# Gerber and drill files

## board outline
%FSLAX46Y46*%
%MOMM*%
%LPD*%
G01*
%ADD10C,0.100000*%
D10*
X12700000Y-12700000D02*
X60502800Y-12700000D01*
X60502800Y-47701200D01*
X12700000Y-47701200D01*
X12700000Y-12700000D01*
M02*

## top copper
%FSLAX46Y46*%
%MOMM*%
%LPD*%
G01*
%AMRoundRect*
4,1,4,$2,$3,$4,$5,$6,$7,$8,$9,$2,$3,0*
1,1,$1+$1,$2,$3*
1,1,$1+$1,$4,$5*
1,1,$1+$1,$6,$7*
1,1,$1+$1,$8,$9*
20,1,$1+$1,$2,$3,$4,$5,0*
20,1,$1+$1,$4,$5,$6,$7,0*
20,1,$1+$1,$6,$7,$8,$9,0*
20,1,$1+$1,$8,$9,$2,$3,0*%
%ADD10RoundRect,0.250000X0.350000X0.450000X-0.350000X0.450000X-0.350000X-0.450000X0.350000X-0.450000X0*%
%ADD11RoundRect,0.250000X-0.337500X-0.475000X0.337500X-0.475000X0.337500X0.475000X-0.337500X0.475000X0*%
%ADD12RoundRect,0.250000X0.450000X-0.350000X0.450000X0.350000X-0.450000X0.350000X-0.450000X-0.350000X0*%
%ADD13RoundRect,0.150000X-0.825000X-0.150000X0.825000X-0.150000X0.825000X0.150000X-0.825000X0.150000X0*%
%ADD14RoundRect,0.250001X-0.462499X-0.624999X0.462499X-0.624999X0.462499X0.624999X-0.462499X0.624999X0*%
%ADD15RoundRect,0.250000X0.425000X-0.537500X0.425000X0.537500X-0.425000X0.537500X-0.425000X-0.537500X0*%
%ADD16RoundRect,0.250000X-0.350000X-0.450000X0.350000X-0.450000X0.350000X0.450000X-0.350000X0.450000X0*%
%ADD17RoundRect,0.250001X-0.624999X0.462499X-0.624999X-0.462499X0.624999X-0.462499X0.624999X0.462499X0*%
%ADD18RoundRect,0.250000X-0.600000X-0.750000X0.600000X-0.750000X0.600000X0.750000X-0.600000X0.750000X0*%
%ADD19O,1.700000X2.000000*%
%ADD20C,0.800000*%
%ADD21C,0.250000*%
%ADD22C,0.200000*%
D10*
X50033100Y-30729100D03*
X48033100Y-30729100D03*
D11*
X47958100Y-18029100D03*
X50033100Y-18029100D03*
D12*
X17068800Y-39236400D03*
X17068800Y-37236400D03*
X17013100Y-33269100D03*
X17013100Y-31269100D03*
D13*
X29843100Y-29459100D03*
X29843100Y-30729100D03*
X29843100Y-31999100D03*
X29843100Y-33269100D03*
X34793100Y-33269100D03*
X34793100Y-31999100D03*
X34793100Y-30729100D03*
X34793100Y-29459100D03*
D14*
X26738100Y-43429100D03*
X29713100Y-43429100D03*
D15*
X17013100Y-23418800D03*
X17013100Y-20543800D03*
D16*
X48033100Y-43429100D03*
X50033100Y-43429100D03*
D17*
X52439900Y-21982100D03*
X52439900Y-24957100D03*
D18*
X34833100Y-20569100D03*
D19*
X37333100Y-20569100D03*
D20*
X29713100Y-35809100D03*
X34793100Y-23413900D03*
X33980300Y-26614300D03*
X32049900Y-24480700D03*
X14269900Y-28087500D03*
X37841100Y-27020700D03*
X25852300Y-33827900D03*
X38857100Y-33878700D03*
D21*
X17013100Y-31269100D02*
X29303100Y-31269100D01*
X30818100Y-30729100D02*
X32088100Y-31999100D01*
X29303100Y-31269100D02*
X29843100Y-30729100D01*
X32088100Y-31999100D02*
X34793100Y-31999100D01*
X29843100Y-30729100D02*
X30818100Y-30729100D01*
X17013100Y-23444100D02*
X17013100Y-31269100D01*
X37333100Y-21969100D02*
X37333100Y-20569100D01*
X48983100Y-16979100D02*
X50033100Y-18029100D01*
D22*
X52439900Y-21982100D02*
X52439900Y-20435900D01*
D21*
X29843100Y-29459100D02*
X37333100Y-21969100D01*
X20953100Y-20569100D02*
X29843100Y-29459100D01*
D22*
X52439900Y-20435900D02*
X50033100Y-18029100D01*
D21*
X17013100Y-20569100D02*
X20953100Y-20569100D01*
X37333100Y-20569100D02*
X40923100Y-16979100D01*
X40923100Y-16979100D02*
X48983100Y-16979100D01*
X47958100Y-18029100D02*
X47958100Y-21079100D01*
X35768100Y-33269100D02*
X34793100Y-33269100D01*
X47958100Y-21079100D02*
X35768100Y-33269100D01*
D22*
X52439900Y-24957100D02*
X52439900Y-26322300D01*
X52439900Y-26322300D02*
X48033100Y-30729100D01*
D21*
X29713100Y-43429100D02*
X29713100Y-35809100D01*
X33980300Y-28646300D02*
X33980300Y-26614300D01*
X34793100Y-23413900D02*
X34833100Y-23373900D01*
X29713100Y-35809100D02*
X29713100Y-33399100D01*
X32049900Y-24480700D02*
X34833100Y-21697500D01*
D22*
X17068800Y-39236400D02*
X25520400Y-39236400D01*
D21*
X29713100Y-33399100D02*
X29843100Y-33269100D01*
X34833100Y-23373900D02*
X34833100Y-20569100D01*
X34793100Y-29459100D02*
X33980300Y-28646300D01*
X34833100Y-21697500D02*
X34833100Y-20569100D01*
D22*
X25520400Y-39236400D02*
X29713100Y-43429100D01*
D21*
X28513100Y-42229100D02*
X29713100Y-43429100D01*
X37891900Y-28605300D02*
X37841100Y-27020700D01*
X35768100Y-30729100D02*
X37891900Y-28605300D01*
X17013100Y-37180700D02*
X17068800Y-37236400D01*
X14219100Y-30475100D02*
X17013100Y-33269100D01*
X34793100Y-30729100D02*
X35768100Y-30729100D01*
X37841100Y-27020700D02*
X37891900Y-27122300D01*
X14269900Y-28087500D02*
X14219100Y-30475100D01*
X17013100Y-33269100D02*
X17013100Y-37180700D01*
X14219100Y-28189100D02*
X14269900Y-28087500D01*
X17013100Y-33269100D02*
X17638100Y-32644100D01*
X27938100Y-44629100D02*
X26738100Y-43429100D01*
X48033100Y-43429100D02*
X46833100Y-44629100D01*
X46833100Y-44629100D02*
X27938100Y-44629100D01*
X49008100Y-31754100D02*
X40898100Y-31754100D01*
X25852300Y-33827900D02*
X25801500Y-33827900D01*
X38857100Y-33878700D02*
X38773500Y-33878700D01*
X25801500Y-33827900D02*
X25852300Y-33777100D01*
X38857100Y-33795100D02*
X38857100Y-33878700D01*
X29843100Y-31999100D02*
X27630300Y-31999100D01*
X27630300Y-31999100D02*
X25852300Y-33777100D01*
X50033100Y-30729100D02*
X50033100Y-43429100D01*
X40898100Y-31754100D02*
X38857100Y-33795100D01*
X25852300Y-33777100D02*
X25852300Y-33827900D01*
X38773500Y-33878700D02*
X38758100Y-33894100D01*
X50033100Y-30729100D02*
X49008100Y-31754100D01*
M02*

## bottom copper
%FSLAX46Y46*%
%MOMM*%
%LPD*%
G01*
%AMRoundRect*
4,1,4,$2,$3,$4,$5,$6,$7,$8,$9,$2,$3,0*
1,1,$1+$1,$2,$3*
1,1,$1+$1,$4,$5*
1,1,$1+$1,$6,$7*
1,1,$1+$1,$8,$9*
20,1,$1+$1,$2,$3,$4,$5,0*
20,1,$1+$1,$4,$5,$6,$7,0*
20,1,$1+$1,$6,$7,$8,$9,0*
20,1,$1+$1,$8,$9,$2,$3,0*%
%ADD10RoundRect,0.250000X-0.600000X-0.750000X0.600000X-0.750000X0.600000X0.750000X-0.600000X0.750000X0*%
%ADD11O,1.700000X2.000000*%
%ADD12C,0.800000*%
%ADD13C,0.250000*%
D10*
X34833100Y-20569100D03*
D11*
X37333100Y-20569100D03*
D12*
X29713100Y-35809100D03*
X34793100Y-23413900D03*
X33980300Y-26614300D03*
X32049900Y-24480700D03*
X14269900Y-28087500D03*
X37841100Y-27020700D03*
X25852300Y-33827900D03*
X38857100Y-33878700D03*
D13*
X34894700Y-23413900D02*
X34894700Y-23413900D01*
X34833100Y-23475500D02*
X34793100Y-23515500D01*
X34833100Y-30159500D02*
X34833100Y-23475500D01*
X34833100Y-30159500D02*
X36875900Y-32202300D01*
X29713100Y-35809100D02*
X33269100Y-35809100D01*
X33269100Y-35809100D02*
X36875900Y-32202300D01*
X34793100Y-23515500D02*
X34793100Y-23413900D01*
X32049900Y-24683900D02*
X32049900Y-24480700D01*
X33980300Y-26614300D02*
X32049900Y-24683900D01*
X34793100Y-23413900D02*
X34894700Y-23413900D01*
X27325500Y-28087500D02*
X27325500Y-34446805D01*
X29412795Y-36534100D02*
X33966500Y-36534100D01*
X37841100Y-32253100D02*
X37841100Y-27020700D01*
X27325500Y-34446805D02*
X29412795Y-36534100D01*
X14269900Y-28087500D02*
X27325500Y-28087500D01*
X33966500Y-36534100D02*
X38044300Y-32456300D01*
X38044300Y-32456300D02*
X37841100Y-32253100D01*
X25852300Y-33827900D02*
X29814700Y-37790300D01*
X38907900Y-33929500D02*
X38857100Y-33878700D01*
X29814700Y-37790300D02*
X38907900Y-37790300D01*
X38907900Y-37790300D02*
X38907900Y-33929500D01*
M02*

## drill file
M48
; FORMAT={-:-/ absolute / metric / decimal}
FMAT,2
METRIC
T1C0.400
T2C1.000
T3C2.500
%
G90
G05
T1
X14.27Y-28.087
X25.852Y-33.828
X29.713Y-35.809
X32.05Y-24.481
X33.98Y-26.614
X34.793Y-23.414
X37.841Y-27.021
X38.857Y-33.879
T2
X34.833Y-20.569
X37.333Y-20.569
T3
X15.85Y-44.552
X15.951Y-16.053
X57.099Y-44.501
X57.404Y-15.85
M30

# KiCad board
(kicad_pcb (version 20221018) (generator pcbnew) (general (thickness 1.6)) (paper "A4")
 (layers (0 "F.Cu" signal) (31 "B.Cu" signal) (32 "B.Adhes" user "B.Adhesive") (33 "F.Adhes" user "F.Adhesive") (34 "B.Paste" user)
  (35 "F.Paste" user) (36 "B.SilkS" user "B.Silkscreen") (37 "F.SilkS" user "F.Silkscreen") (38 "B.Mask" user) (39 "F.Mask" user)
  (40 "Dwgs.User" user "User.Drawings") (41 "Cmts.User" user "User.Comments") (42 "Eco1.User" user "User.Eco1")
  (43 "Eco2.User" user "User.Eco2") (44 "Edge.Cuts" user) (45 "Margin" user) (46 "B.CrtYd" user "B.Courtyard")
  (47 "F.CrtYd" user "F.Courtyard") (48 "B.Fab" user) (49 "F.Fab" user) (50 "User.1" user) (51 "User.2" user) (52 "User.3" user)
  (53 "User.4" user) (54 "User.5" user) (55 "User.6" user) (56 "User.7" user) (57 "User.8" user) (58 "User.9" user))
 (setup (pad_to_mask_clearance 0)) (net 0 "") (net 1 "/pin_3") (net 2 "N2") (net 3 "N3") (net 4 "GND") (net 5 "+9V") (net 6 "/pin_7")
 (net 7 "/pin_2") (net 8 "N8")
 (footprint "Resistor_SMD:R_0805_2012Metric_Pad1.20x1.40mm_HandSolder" (layer "F.Cu") (at 49.0331 30.7291 180)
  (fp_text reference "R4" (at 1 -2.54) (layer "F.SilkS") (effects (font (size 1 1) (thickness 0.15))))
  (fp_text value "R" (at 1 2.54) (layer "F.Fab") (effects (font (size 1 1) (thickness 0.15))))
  (pad "1" smd roundrect (at -1 0 180) (size 1.2 1.4) (layers "F.Cu" "F.Paste" "F.Mask") (roundrect_rratio 0.208333) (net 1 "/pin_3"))
  (pad "2" smd roundrect (at 1 0 180) (size 1.2 1.4) (layers "F.Cu" "F.Paste" "F.Mask") (roundrect_rratio 0.208333) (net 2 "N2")))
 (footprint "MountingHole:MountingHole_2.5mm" (layer "F.Cu") (at 15.8496 44.5516)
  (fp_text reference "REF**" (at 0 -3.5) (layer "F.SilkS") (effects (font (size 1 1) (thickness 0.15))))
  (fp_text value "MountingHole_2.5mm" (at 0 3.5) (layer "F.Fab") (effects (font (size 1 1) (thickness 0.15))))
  (pad "" np_thru_hole circle (at 0 0) (size 2.5 2.5) (drill 2.5) (layers "*.Cu" "*.Mask")))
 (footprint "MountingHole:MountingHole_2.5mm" (layer "F.Cu") (at 57.0992 44.5008)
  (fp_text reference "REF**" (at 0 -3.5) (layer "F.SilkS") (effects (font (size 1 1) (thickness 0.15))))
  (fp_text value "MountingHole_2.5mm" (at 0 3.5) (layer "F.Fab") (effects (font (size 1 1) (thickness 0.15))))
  (pad "" np_thru_hole circle (at 0 0) (size 2.5 2.5) (drill 2.5) (layers "*.Cu" "*.Mask")))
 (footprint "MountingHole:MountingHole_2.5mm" (layer "F.Cu") (at 15.9512 16.0528)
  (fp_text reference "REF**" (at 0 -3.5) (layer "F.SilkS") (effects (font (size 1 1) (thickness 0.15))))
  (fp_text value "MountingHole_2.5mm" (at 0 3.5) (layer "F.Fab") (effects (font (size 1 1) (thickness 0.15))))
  (pad "" np_thru_hole circle (at 0 0) (size 2.5 2.5) (drill 2.5) (layers "*.Cu" "*.Mask")))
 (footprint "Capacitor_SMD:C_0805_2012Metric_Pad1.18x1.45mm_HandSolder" (layer "F.Cu") (at 48.9956 18.0291)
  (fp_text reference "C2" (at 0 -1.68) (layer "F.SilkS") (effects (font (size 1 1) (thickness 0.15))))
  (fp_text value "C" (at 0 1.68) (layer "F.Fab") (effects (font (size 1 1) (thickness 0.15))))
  (pad "1" smd roundrect (at -1.0375 0) (size 1.175 1.45) (layers "F.Cu" "F.Paste" "F.Mask") (roundrect_rratio 0.212766) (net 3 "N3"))
  (pad "2" smd roundrect (at 1.0375 0) (size 1.175 1.45) (layers "F.Cu" "F.Paste" "F.Mask") (roundrect_rratio 0.212766) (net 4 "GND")))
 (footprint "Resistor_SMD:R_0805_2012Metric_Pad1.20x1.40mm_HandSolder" (layer "F.Cu") (at 17.0688 38.2364 90)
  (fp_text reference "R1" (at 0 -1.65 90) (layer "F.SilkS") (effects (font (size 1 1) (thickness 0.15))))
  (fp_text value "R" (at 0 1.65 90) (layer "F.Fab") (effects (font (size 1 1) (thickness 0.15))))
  (pad "1" smd roundrect (at -1 0 90) (size 1.2 1.4) (layers "F.Cu" "F.Paste" "F.Mask") (roundrect_rratio 0.208333) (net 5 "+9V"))
  (pad "2" smd roundrect (at 1 0 90) (size 1.2 1.4) (layers "F.Cu" "F.Paste" "F.Mask") (roundrect_rratio 0.208333) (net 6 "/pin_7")))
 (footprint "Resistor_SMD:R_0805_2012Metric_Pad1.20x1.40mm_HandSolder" (layer "F.Cu") (at 17.0131 32.2691 90)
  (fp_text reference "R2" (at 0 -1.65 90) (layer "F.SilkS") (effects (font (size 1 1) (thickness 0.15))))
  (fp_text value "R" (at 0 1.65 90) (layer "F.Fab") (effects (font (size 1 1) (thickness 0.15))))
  (pad "1" smd roundrect (at -1 0 90) (size 1.2 1.4) (layers "F.Cu" "F.Paste" "F.Mask") (roundrect_rratio 0.208333) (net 6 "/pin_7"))
  (pad "2" smd roundrect (at 1 0 90) (size 1.2 1.4) (layers "F.Cu" "F.Paste" "F.Mask") (roundrect_rratio 0.208333) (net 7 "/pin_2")))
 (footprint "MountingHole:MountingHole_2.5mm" (layer "F.Cu") (at 57.404 15.8496)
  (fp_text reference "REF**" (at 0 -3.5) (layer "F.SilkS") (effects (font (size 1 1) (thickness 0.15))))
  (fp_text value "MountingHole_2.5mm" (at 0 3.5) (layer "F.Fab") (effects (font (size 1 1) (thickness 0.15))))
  (pad "" np_thru_hole circle (at 0 0) (size 2.5 2.5) (drill 2.5) (layers "*.Cu" "*.Mask")))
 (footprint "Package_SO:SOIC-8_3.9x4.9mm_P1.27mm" (layer "F.Cu") (at 32.3181 31.3641)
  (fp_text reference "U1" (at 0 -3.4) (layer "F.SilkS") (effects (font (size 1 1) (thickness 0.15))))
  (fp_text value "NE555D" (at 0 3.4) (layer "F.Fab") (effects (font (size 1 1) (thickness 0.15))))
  (pad "1" smd roundrect (at -2.475 -1.905) (size 1.95 0.6) (layers "F.Cu" "F.Paste" "F.Mask") (roundrect_rratio 0.25) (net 4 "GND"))
  (pad "2" smd roundrect (at -2.475 -0.635) (size 1.95 0.6) (layers "F.Cu" "F.Paste" "F.Mask") (roundrect_rratio 0.25) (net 7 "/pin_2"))
  (pad "3" smd roundrect (at -2.475 0.635) (size 1.95 0.6) (layers "F.Cu" "F.Paste" "F.Mask") (roundrect_rratio 0.25) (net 1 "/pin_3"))
  (pad "4" smd roundrect (at -2.475 1.905) (size 1.95 0.6) (layers "F.Cu" "F.Paste" "F.Mask") (roundrect_rratio 0.25) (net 5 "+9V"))
  (pad "5" smd roundrect (at 2.475 1.905) (size 1.95 0.6) (layers "F.Cu" "F.Paste" "F.Mask") (roundrect_rratio 0.25) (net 3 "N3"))
  (pad "6" smd roundrect (at 2.475 0.635) (size 1.95 0.6) (layers "F.Cu" "F.Paste" "F.Mask") (roundrect_rratio 0.25) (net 7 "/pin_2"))
  (pad "7" smd roundrect (at 2.475 -0.635) (size 1.95 0.6) (layers "F.Cu" "F.Paste" "F.Mask") (roundrect_rratio 0.25) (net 6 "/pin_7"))
  (pad "8" smd roundrect (at 2.475 -1.905) (size 1.95 0.6) (layers "F.Cu" "F.Paste" "F.Mask") (roundrect_rratio 0.25) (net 5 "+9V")))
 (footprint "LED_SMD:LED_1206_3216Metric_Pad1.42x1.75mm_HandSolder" (layer "F.Cu") (at 28.2256 43.4291)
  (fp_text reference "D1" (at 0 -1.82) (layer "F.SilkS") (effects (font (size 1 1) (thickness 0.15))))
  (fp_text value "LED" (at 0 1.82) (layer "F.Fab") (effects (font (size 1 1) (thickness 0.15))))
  (pad "1" smd roundrect (at -1.4875 0) (size 1.425 1.75) (layers "F.Cu" "F.Paste" "F.Mask") (roundrect_rratio 0.175439) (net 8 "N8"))
  (pad "2" smd roundrect (at 1.4875 0) (size 1.425 1.75) (layers "F.Cu" "F.Paste" "F.Mask") (roundrect_rratio 0.175439) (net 5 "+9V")))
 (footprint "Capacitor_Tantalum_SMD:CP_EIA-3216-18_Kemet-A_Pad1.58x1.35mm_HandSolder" (layer "F.Cu") (at 17.0131 21.9813 90)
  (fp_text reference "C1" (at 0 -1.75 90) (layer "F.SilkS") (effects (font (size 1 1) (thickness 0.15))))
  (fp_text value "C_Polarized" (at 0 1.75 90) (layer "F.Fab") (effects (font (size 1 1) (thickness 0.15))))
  (pad "1" smd roundrect (at -1.4375 0 90) (size 1.575 1.35) (layers "F.Cu" "F.Paste" "F.Mask") (roundrect_rratio 0.185185) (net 7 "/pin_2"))
  (pad "2" smd roundrect (at 1.4375 0 90) (size 1.575 1.35) (layers "F.Cu" "F.Paste" "F.Mask") (roundrect_rratio 0.185185) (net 4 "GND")))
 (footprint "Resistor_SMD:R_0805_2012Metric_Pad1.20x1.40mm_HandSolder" (layer "F.Cu") (at 49.0331 43.4291)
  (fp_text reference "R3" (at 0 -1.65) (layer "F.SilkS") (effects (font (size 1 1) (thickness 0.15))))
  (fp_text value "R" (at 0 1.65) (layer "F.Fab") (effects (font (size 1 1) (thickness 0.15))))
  (pad "1" smd roundrect (at -1 0) (size 1.2 1.4) (layers "F.Cu" "F.Paste" "F.Mask") (roundrect_rratio 0.208333) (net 8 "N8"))
  (pad "2" smd roundrect (at 1 0) (size 1.2 1.4) (layers "F.Cu" "F.Paste" "F.Mask") (roundrect_rratio 0.208333) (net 1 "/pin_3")))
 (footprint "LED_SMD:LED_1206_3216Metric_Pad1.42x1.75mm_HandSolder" (layer "F.Cu") (at 52.4399 23.4696 -90)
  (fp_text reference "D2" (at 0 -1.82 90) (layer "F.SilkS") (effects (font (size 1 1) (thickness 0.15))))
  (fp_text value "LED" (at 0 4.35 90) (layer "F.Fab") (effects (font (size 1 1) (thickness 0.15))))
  (pad "1" smd roundrect (at -1.4875 0 270) (size 1.425 1.75) (layers "F.Cu" "F.Paste" "F.Mask") (roundrect_rratio 0.175439) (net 4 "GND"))
  (pad "2" smd roundrect (at 1.4875 0 270) (size 1.425 1.75) (layers "F.Cu" "F.Paste" "F.Mask") (roundrect_rratio 0.175439) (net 2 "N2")))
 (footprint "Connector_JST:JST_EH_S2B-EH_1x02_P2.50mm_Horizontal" (layer "F.Cu") (at 34.8331 20.5691)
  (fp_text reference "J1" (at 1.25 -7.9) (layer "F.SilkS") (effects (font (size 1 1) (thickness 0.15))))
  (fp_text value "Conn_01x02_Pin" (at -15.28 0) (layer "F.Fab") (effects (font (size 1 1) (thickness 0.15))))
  (pad "1" thru_hole roundrect (at 0 0) (size 1.7 2) (drill 1) (layers "*.Cu" "*.Mask") (roundrect_rratio 0.147059) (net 5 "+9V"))
  (pad "2" thru_hole oval (at 2.5 0) (size 1.7 2) (drill 1) (layers "*.Cu" "*.Mask") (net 4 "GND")))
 (gr_rect (start 12.7 12.7) (end 60.5028 47.7012) (stroke (width 0.1) (type default)) (fill none) (layer "Edge.Cuts"))
 (segment (start 17.0131 31.2691) (end 29.3031 31.2691) (width 0.25) (layer "F.Cu") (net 7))
 (segment (start 30.8181 30.7291) (end 32.0881 31.9991) (width 0.25) (layer "F.Cu") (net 7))
 (segment (start 29.3031 31.2691) (end 29.8431 30.7291) (width 0.25) (layer "F.Cu") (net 7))
 (segment (start 32.0881 31.9991) (end 34.7931 31.9991) (width 0.25) (layer "F.Cu") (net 7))
 (segment (start 29.8431 30.7291) (end 30.8181 30.7291) (width 0.25) (layer "F.Cu") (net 7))
 (segment (start 17.0131 23.4441) (end 17.0131 31.2691) (width 0.25) (layer "F.Cu") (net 7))
 (segment (start 37.3331 21.9691) (end 37.3331 20.5691) (width 0.25) (layer "F.Cu") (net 4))
 (segment (start 48.9831 16.9791) (end 50.0331 18.0291) (width 0.25) (layer "F.Cu") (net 4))
 (segment (start 52.4399 21.9821) (end 52.4399 20.4359) (width 0.2) (layer "F.Cu") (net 4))
 (segment (start 29.8431 29.4591) (end 37.3331 21.9691) (width 0.25) (layer "F.Cu") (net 4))
 (segment (start 20.9531 20.5691) (end 29.8431 29.4591) (width 0.25) (layer "F.Cu") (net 4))
 (segment (start 52.4399 20.4359) (end 50.0331 18.0291) (width 0.2) (layer "F.Cu") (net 4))
 (segment (start 17.0131 20.5691) (end 20.9531 20.5691) (width 0.25) (layer "F.Cu") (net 4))
 (segment (start 37.3331 20.5691) (end 40.9231 16.9791) (width 0.25) (layer "F.Cu") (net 4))
 (segment (start 40.9231 16.9791) (end 48.9831 16.9791) (width 0.25) (layer "F.Cu") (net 4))
 (segment (start 47.9581 18.0291) (end 47.9581 21.0791) (width 0.25) (layer "F.Cu") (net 3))
 (segment (start 35.7681 33.2691) (end 34.7931 33.2691) (width 0.25) (layer "F.Cu") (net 3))
 (segment (start 47.9581 21.0791) (end 35.7681 33.2691) (width 0.25) (layer "F.Cu") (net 3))
 (segment (start 52.4399 24.9571) (end 52.4399 26.3223) (width 0.2) (layer "F.Cu") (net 2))
 (segment (start 52.4399 26.3223) (end 48.0331 30.7291) (width 0.2) (layer "F.Cu") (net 2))
 (segment (start 29.7131 43.4291) (end 29.7131 35.8091) (width 0.25) (layer "F.Cu") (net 5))
 (segment (start 33.9803 28.6463) (end 33.9803 26.6143) (width 0.25) (layer "F.Cu") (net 5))
 (segment (start 34.7931 23.4139) (end 34.8331 23.3739) (width 0.25) (layer "F.Cu") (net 5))
 (segment (start 29.7131 35.8091) (end 29.7131 33.3991) (width 0.25) (layer "F.Cu") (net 5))
 (segment (start 32.0499 24.4807) (end 34.8331 21.6975) (width 0.25) (layer "F.Cu") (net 5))
 (segment (start 17.0688 39.2364) (end 25.5204 39.2364) (width 0.2) (layer "F.Cu") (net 5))
 (segment (start 29.7131 33.3991) (end 29.8431 33.2691) (width 0.25) (layer "F.Cu") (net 5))
 (segment (start 34.8331 23.3739) (end 34.8331 20.5691) (width 0.25) (layer "F.Cu") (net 5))
 (segment (start 34.7931 29.4591) (end 33.9803 28.6463) (width 0.25) (layer "F.Cu") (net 5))
 (segment (start 34.8331 21.6975) (end 34.8331 20.5691) (width 0.25) (layer "F.Cu") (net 5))
 (segment (start 25.5204 39.2364) (end 29.7131 43.4291) (width 0.2) (layer "F.Cu") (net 5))
 (segment (start 28.5131 42.2291) (end 29.7131 43.4291) (width 0.25) (layer "F.Cu") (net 5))
 (via (at 29.7131 35.8091) (size 0.8) (drill 0.4) (layers "F.Cu" "B.Cu") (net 5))
 (via (at 34.7931 23.4139) (size 0.8) (drill 0.4) (layers "F.Cu" "B.Cu") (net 5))
 (via (at 33.9803 26.6143) (size 0.8) (drill 0.4) (layers "F.Cu" "B.Cu") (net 5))
 (via (at 32.0499 24.4807) (size 0.8) (drill 0.4) (layers "F.Cu" "B.Cu") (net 5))
 (segment (start 34.8947 23.4139) (end 34.8947 23.4139) (width 0.25) (layer "B.Cu") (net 5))
 (segment (start 34.8331 23.4755) (end 34.7931 23.5155) (width 0.25) (layer "B.Cu") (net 5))
 (segment (start 34.8331 30.1595) (end 34.8331 23.4755) (width 0.25) (layer "B.Cu") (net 5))
 (segment (start 34.8331 30.1595) (end 36.8759 32.2023) (width 0.25) (layer "B.Cu") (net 5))
 (segment (start 29.7131 35.8091) (end 33.2691 35.8091) (width 0.25) (layer "B.Cu") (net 5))
 (segment (start 33.2691 35.8091) (end 36.8759 32.2023) (width 0.25) (layer "B.Cu") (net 5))
 (segment (start 34.7931 23.5155) (end 34.7931 23.4139) (width 0.25) (layer "B.Cu") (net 5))
 (segment (start 32.0499 24.6839) (end 32.0499 24.4807) (width 0.25) (layer "B.Cu") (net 5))
 (segment (start 33.9803 26.6143) (end 32.0499 24.6839) (width 0.25) (layer "B.Cu") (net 5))
 (segment (start 34.7931 23.4139) (end 34.8947 23.4139) (width 0.25) (layer "B.Cu") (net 5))
 (segment (start 37.8919 28.6053) (end 37.8411 27.0207) (width 0.25) (layer "F.Cu") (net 6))
 (segment (start 35.7681 30.7291) (end 37.8919 28.6053) (width 0.25) (layer "F.Cu") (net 6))
 (segment (start 17.0131 37.1807) (end 17.0688 37.2364) (width 0.25) (layer "F.Cu") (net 6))
 (segment (start 14.2191 30.4751) (end 17.0131 33.2691) (width 0.25) (layer "F.Cu") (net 6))
 (segment (start 34.7931 30.7291) (end 35.7681 30.7291) (width 0.25) (layer "F.Cu") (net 6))
 (segment (start 37.8411 27.0207) (end 37.8919 27.1223) (width 0.25) (layer "F.Cu") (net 6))
 (segment (start 14.2699 28.0875) (end 14.2191 30.4751) (width 0.25) (layer "F.Cu") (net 6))
 (segment (start 17.0131 33.2691) (end 17.0131 37.1807) (width 0.25) (layer "F.Cu") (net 6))
 (segment (start 14.2191 28.1891) (end 14.2699 28.0875) (width 0.25) (layer "F.Cu") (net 6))
 (segment (start 17.0131 33.2691) (end 17.6381 32.6441) (width 0.25) (layer "F.Cu") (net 6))
 (via (at 14.2699 28.0875) (size 0.8) (drill 0.4) (layers "F.Cu" "B.Cu") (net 6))
 (via (at 37.8411 27.0207) (size 0.8) (drill 0.4) (layers "F.Cu" "B.Cu") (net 6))
 (segment (start 27.3255 28.0875) (end 27.3255 34.446805) (width 0.25) (layer "B.Cu") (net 6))
 (segment (start 29.412795 36.5341) (end 33.9665 36.5341) (width 0.25) (layer "B.Cu") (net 6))
 (segment (start 37.8411 32.2531) (end 37.8411 27.0207) (width 0.25) (layer "B.Cu") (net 6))
 (segment (start 27.3255 34.446805) (end 29.412795 36.5341) (width 0.25) (layer "B.Cu") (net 6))
 (segment (start 14.2699 28.0875) (end 27.3255 28.0875) (width 0.25) (layer "B.Cu") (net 6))
 (segment (start 33.9665 36.5341) (end 38.0443 32.4563) (width 0.25) (layer "B.Cu") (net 6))
 (segment (start 38.0443 32.4563) (end 37.8411 32.2531) (width 0.25) (layer "B.Cu") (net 6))
 (segment (start 27.9381 44.6291) (end 26.7381 43.4291) (width 0.25) (layer "F.Cu") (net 8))
 (segment (start 48.0331 43.4291) (end 46.8331 44.6291) (width 0.25) (layer "F.Cu") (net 8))
 (segment (start 46.8331 44.6291) (end 27.9381 44.6291) (width 0.25) (layer "F.Cu") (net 8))
 (segment (start 49.0081 31.7541) (end 40.8981 31.7541) (width 0.25) (layer "F.Cu") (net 1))
 (segment (start 25.8523 33.8279) (end 25.8015 33.8279) (width 0.25) (layer "F.Cu") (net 1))
 (segment (start 38.8571 33.8787) (end 38.7735 33.8787) (width 0.25) (layer "F.Cu") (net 1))
 (segment (start 25.8015 33.8279) (end 25.8523 33.7771) (width 0.25) (layer "F.Cu") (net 1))
 (segment (start 38.8571 33.7951) (end 38.8571 33.8787) (width 0.25) (layer "F.Cu") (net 1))
 (segment (start 29.8431 31.9991) (end 27.6303 31.9991) (width 0.25) (layer "F.Cu") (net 1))
 (segment (start 27.6303 31.9991) (end 25.8523 33.7771) (width 0.25) (layer "F.Cu") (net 1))
 (segment (start 50.0331 30.7291) (end 50.0331 43.4291) (width 0.25) (layer "F.Cu") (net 1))
 (segment (start 40.8981 31.7541) (end 38.8571 33.7951) (width 0.25) (layer "F.Cu") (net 1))
 (segment (start 25.8523 33.7771) (end 25.8523 33.8279) (width 0.25) (layer "F.Cu") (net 1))
 (segment (start 38.7735 33.8787) (end 38.7581 33.8941) (width 0.25) (layer "F.Cu") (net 1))
 (segment (start 50.0331 30.7291) (end 49.0081 31.7541) (width 0.25) (layer "F.Cu") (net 1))
 (via (at 25.8523 33.8279) (size 0.8) (drill 0.4) (layers "F.Cu" "B.Cu") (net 1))
 (via (at 38.8571 33.8787) (size 0.8) (drill 0.4) (layers "F.Cu" "B.Cu") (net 1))
 (segment (start 25.8523 33.8279) (end 29.8147 37.7903) (width 0.25) (layer "B.Cu") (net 1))
 (segment (start 38.9079 33.9295) (end 38.8571 33.8787) (width 0.25) (layer "B.Cu") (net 1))
 (segment (start 29.8147 37.7903) (end 38.9079 37.7903) (width 0.25) (layer "B.Cu") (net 1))
 (segment (start 38.9079 37.7903) (end 38.9079 33.9295) (width 0.25) (layer "B.Cu") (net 1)))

